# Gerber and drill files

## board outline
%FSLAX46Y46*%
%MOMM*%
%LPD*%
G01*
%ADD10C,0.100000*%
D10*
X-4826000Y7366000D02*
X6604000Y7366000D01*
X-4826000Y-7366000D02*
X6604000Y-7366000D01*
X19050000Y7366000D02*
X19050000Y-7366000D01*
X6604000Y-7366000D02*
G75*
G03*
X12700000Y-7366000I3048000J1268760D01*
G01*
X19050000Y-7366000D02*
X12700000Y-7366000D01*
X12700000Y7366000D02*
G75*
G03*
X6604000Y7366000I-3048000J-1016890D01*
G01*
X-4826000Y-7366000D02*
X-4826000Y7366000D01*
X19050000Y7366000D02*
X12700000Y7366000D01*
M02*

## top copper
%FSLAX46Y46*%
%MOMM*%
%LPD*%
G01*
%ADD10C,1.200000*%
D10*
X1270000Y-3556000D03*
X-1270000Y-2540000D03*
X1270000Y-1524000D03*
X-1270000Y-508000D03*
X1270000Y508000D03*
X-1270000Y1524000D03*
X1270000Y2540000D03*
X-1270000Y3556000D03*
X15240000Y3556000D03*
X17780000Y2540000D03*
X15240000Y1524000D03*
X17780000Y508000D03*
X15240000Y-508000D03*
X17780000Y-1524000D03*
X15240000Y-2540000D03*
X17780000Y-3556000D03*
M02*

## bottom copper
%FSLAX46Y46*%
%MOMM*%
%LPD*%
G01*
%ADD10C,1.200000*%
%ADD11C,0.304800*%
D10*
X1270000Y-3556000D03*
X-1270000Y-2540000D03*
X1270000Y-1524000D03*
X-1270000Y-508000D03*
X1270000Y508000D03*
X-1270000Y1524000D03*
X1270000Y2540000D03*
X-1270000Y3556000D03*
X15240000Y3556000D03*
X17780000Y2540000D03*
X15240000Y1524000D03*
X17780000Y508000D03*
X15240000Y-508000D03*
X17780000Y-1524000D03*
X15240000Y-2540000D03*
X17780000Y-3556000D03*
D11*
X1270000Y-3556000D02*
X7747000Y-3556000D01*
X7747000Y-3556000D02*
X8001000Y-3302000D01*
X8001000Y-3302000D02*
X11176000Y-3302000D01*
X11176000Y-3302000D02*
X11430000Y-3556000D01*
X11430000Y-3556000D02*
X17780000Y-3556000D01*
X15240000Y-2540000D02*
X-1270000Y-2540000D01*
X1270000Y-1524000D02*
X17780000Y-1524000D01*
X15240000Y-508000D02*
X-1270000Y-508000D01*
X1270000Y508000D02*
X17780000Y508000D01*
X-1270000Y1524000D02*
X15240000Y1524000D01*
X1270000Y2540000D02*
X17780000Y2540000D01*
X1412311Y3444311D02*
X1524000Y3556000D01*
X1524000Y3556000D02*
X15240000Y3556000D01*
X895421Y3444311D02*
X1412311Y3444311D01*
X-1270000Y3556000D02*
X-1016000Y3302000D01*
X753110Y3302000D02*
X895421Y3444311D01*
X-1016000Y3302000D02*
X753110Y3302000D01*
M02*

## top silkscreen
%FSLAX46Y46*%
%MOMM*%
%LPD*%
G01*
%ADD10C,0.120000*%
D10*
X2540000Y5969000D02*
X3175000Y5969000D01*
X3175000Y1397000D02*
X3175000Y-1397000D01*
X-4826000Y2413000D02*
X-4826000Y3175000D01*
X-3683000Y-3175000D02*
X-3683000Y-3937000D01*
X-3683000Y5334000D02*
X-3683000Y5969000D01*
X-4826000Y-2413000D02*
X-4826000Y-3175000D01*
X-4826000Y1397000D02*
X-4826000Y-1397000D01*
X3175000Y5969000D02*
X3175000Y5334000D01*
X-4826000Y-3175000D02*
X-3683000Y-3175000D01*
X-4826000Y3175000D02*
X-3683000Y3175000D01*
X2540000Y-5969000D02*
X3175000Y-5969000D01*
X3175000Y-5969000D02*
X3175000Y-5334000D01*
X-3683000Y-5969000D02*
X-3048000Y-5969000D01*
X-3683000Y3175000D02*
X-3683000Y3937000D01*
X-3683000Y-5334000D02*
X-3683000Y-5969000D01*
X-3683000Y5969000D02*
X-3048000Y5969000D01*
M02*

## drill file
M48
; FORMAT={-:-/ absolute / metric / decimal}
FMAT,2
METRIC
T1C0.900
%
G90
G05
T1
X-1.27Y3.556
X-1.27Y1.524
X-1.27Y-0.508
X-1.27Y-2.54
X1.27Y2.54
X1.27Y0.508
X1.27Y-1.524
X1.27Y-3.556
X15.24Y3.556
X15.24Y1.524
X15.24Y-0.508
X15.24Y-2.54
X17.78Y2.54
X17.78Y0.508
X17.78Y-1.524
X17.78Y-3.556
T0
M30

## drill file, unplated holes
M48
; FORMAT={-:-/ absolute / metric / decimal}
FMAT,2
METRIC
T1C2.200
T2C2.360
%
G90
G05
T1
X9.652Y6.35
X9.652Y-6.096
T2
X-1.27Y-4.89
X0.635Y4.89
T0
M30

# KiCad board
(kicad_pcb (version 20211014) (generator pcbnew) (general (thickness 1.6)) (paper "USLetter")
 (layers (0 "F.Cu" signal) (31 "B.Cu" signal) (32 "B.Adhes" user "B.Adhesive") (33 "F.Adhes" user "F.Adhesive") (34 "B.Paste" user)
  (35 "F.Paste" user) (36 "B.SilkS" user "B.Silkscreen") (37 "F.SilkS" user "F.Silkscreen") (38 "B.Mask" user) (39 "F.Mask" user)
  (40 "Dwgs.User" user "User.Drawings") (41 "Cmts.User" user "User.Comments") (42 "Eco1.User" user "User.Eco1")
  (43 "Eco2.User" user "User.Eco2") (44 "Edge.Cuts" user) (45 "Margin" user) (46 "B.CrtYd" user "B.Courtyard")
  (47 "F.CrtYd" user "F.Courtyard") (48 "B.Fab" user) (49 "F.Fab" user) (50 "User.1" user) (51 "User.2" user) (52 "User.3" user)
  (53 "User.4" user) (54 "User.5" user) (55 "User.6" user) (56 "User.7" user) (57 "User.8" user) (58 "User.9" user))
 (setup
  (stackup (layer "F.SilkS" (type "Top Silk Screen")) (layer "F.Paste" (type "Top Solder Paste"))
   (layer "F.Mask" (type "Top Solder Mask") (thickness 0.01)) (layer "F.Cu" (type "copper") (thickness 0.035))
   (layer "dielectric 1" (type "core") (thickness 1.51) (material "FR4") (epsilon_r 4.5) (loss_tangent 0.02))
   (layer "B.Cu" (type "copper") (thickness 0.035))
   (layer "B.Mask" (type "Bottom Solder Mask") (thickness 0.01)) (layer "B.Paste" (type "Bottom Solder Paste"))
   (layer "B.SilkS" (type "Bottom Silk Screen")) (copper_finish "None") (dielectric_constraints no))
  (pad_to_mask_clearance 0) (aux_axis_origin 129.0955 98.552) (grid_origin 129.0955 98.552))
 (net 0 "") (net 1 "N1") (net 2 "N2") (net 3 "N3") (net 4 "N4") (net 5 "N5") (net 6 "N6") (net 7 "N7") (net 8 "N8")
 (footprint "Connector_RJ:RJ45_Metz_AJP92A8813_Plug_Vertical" (layer "F.Cu") (at 129.0955 98.552 90)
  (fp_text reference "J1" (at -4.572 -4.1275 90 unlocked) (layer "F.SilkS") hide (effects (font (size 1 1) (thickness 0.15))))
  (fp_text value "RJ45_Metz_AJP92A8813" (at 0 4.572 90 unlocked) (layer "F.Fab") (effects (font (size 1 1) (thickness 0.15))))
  (fp_line (start 5.969 2.54) (end 5.969 3.175) (layer "F.SilkS") (width 0.12))
  (fp_line (start 1.397 3.175) (end -1.397 3.175) (layer "F.SilkS") (width 0.12))
  (fp_line (start 2.413 -4.826) (end 3.175 -4.826) (layer "F.SilkS") (width 0.12))
  (fp_line (start -3.175 -3.683) (end -3.937 -3.683) (layer "F.SilkS") (width 0.12))
  (fp_line (start 5.334 -3.683) (end 5.969 -3.683) (layer "F.SilkS") (width 0.12))
  (fp_line (start -2.413 -4.826) (end -3.175 -4.826) (layer "F.SilkS") (width 0.12))
  (fp_line (start 1.397 -4.826) (end -1.397 -4.826) (layer "F.SilkS") (width 0.12))
  (fp_line (start 5.969 3.175) (end 5.334 3.175) (layer "F.SilkS") (width 0.12))
  (fp_line (start -3.175 -4.826) (end -3.175 -3.683) (layer "F.SilkS") (width 0.12))
  (fp_line (start 3.175 -4.826) (end 3.175 -3.683) (layer "F.SilkS") (width 0.12))
  (fp_line (start -5.969 2.54) (end -5.969 3.175) (layer "F.SilkS") (width 0.12))
  (fp_line (start -5.969 3.175) (end -5.334 3.175) (layer "F.SilkS") (width 0.12))
  (fp_line (start -5.969 -3.683) (end -5.969 -3.048) (layer "F.SilkS") (width 0.12))
  (fp_line (start 3.175 -3.683) (end 3.937 -3.683) (layer "F.SilkS") (width 0.12))
  (fp_line (start -5.334 -3.683) (end -5.969 -3.683) (layer "F.SilkS") (width 0.12))
  (fp_line (start 5.969 -3.683) (end 5.969 -3.048) (layer "F.SilkS") (width 0.12))
  (pad "" np_thru_hole circle (at -4.89 -1.27 90) (size 2.36 2.36) (drill 2.36) (layers *.Mask))
  (pad "" np_thru_hole circle (at 4.89 0.635 90) (size 2.36 2.36) (drill 2.36) (layers *.Mask))
  (pad "1" thru_hole circle (at -3.556 1.27 90) (size 1.2 1.2) (drill 0.9) (layers *.Cu *.Mask) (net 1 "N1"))
  (pad "2" thru_hole circle (at -2.54 -1.27 90) (size 1.2 1.2) (drill 0.9) (layers *.Cu *.Mask) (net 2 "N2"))
  (pad "3" thru_hole circle (at -1.524 1.27 90) (size 1.2 1.2) (drill 0.9) (layers *.Cu *.Mask) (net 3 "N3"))
  (pad "4" thru_hole circle (at -0.508 -1.27 90) (size 1.2 1.2) (drill 0.9) (layers *.Cu *.Mask) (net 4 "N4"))
  (pad "5" thru_hole circle (at 0.508 1.27 90) (size 1.2 1.2) (drill 0.9) (layers *.Cu *.Mask) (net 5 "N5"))
  (pad "6" thru_hole circle (at 1.524 -1.27 90) (size 1.2 1.2) (drill 0.9) (layers *.Cu *.Mask) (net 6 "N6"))
  (pad "7" thru_hole circle (at 2.54 1.27 90) (size 1.2 1.2) (drill 0.9) (layers *.Cu *.Mask) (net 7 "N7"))
  (pad "8" thru_hole circle (at 3.556 -1.27 90) (size 1.2 1.2) (drill 0.9) (layers *.Cu *.Mask) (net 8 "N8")))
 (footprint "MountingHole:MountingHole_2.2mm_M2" (layer "F.Cu") (at 138.7475 92.202)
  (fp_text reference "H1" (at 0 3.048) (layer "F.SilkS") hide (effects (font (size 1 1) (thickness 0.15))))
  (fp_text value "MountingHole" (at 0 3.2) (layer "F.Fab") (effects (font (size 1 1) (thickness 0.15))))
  (pad "" np_thru_hole circle (at 0 0) (size 2.2 2.2) (drill 2.2) (layers *.Cu *.Mask)))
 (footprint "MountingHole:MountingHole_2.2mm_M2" (layer "F.Cu") (at 138.7475 104.648)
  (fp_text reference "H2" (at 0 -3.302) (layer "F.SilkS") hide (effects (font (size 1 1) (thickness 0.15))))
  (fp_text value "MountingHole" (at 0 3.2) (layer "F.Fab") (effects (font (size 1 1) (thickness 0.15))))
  (pad "" np_thru_hole circle (at 0 0) (size 2.2 2.2) (drill 2.2) (layers *.Cu *.Mask)))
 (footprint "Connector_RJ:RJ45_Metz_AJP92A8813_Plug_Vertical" (layer "F.Cu") (at 145.6055 98.552 -90)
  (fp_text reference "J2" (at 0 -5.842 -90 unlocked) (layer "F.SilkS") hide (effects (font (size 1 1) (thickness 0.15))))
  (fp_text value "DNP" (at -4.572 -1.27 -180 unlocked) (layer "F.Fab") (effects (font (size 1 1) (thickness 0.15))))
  (pad "1" thru_hole circle (at -3.556 1.27 270) (size 1.2 1.2) (drill 0.9) (layers *.Cu *.Mask) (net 8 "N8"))
  (pad "2" thru_hole circle (at -2.54 -1.27 270) (size 1.2 1.2) (drill 0.9) (layers *.Cu *.Mask) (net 7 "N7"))
  (pad "3" thru_hole circle (at -1.524 1.27 270) (size 1.2 1.2) (drill 0.9) (layers *.Cu *.Mask) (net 6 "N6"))
  (pad "4" thru_hole circle (at -0.508 -1.27 270) (size 1.2 1.2) (drill 0.9) (layers *.Cu *.Mask) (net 5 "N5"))
  (pad "5" thru_hole circle (at 0.508 1.27 270) (size 1.2 1.2) (drill 0.9) (layers *.Cu *.Mask) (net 4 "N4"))
  (pad "6" thru_hole circle (at 1.524 -1.27 270) (size 1.2 1.2) (drill 0.9) (layers *.Cu *.Mask) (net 3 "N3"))
  (pad "7" thru_hole circle (at 2.54 1.27 270) (size 1.2 1.2) (drill 0.9) (layers *.Cu *.Mask) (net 2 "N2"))
  (pad "8" thru_hole circle (at 3.556 -1.27 270) (size 1.2 1.2) (drill 0.9) (layers *.Cu *.Mask) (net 1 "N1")))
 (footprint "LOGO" (layer "B.Cu") (at 137.871545 103.684672 90)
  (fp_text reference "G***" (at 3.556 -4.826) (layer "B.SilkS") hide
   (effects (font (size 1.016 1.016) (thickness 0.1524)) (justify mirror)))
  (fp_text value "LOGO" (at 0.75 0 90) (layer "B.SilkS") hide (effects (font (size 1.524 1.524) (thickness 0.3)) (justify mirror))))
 (gr_line (start 124.2695 91.186) (end 135.6995 91.186) (layer "Edge.Cuts") (width 0.1))
 (gr_line (start 124.2695 105.918) (end 135.6995 105.918) (layer "Edge.Cuts") (width 0.1))
 (gr_line (start 148.1455 91.186) (end 148.1455 105.918) (layer "Edge.Cuts") (width 0.1))
 (gr_arc (start 141.7955 105.918) (mid 138.7475 107.950763) (end 135.6995 105.918) (layer "Edge.Cuts") (width 0.1))
 (gr_line (start 148.1455 105.918) (end 141.7955 105.918) (layer "Edge.Cuts") (width 0.1))
 (gr_arc (start 135.6995 91.186) (mid 138.7475 88.989734) (end 141.7955 91.186) (layer "Edge.Cuts") (width 0.1))
 (gr_line (start 124.2695 105.918) (end 124.2695 91.186) (layer "Edge.Cuts") (width 0.1))
 (gr_line (start 148.1455 91.186) (end 141.7955 91.186) (layer "Edge.Cuts") (width 0.1))
 (segment (start 140.2715 101.854) (end 140.5255 102.108) (width 0.3048) (layer "B.Cu") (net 1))
 (segment (start 140.5255 102.108) (end 146.8755 102.108) (width 0.3048) (layer "B.Cu") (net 1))
 (segment (start 136.8425 102.108) (end 137.0965 101.854) (width 0.3048) (layer "B.Cu") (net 1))
 (segment (start 130.3655 102.108) (end 136.8425 102.108) (width 0.3048) (layer "B.Cu") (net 1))
 (segment (start 137.0965 101.854) (end 140.2715 101.854) (width 0.3048) (layer "B.Cu") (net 1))
 (segment (start 144.3355 101.092) (end 127.8255 101.092) (width 0.3048) (layer "B.Cu") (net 2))
 (segment (start 130.3655 100.076) (end 146.8755 100.076) (width 0.3048) (layer "B.Cu") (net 3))
 (segment (start 144.3355 99.06) (end 127.8255 99.06) (width 0.3048) (layer "B.Cu") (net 4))
 (segment (start 130.3655 98.044) (end 146.8755 98.044) (width 0.3048) (layer "B.Cu") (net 5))
 (segment (start 127.8255 97.028) (end 144.3355 97.028) (width 0.3048) (layer "B.Cu") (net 6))
 (segment (start 130.3655 96.012) (end 146.8755 96.012) (width 0.3048) (layer "B.Cu") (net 7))
 (segment (start 130.507811 95.107689) (end 130.6195 94.996) (width 0.3048) (layer "B.Cu") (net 8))
 (segment (start 130.6195 94.996) (end 144.3355 94.996) (width 0.3048) (layer "B.Cu") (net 8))
 (segment (start 129.990921 95.107689) (end 130.507811 95.107689) (width 0.3048) (layer "B.Cu") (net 8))
 (segment (start 127.8255 94.996) (end 128.0795 95.25) (width 0.3048) (layer "B.Cu") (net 8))
 (segment (start 129.84861 95.25) (end 129.990921 95.107689) (width 0.3048) (layer "B.Cu") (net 8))
 (segment (start 128.0795 95.25) (end 129.84861 95.25) (width 0.3048) (layer "B.Cu") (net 8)))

